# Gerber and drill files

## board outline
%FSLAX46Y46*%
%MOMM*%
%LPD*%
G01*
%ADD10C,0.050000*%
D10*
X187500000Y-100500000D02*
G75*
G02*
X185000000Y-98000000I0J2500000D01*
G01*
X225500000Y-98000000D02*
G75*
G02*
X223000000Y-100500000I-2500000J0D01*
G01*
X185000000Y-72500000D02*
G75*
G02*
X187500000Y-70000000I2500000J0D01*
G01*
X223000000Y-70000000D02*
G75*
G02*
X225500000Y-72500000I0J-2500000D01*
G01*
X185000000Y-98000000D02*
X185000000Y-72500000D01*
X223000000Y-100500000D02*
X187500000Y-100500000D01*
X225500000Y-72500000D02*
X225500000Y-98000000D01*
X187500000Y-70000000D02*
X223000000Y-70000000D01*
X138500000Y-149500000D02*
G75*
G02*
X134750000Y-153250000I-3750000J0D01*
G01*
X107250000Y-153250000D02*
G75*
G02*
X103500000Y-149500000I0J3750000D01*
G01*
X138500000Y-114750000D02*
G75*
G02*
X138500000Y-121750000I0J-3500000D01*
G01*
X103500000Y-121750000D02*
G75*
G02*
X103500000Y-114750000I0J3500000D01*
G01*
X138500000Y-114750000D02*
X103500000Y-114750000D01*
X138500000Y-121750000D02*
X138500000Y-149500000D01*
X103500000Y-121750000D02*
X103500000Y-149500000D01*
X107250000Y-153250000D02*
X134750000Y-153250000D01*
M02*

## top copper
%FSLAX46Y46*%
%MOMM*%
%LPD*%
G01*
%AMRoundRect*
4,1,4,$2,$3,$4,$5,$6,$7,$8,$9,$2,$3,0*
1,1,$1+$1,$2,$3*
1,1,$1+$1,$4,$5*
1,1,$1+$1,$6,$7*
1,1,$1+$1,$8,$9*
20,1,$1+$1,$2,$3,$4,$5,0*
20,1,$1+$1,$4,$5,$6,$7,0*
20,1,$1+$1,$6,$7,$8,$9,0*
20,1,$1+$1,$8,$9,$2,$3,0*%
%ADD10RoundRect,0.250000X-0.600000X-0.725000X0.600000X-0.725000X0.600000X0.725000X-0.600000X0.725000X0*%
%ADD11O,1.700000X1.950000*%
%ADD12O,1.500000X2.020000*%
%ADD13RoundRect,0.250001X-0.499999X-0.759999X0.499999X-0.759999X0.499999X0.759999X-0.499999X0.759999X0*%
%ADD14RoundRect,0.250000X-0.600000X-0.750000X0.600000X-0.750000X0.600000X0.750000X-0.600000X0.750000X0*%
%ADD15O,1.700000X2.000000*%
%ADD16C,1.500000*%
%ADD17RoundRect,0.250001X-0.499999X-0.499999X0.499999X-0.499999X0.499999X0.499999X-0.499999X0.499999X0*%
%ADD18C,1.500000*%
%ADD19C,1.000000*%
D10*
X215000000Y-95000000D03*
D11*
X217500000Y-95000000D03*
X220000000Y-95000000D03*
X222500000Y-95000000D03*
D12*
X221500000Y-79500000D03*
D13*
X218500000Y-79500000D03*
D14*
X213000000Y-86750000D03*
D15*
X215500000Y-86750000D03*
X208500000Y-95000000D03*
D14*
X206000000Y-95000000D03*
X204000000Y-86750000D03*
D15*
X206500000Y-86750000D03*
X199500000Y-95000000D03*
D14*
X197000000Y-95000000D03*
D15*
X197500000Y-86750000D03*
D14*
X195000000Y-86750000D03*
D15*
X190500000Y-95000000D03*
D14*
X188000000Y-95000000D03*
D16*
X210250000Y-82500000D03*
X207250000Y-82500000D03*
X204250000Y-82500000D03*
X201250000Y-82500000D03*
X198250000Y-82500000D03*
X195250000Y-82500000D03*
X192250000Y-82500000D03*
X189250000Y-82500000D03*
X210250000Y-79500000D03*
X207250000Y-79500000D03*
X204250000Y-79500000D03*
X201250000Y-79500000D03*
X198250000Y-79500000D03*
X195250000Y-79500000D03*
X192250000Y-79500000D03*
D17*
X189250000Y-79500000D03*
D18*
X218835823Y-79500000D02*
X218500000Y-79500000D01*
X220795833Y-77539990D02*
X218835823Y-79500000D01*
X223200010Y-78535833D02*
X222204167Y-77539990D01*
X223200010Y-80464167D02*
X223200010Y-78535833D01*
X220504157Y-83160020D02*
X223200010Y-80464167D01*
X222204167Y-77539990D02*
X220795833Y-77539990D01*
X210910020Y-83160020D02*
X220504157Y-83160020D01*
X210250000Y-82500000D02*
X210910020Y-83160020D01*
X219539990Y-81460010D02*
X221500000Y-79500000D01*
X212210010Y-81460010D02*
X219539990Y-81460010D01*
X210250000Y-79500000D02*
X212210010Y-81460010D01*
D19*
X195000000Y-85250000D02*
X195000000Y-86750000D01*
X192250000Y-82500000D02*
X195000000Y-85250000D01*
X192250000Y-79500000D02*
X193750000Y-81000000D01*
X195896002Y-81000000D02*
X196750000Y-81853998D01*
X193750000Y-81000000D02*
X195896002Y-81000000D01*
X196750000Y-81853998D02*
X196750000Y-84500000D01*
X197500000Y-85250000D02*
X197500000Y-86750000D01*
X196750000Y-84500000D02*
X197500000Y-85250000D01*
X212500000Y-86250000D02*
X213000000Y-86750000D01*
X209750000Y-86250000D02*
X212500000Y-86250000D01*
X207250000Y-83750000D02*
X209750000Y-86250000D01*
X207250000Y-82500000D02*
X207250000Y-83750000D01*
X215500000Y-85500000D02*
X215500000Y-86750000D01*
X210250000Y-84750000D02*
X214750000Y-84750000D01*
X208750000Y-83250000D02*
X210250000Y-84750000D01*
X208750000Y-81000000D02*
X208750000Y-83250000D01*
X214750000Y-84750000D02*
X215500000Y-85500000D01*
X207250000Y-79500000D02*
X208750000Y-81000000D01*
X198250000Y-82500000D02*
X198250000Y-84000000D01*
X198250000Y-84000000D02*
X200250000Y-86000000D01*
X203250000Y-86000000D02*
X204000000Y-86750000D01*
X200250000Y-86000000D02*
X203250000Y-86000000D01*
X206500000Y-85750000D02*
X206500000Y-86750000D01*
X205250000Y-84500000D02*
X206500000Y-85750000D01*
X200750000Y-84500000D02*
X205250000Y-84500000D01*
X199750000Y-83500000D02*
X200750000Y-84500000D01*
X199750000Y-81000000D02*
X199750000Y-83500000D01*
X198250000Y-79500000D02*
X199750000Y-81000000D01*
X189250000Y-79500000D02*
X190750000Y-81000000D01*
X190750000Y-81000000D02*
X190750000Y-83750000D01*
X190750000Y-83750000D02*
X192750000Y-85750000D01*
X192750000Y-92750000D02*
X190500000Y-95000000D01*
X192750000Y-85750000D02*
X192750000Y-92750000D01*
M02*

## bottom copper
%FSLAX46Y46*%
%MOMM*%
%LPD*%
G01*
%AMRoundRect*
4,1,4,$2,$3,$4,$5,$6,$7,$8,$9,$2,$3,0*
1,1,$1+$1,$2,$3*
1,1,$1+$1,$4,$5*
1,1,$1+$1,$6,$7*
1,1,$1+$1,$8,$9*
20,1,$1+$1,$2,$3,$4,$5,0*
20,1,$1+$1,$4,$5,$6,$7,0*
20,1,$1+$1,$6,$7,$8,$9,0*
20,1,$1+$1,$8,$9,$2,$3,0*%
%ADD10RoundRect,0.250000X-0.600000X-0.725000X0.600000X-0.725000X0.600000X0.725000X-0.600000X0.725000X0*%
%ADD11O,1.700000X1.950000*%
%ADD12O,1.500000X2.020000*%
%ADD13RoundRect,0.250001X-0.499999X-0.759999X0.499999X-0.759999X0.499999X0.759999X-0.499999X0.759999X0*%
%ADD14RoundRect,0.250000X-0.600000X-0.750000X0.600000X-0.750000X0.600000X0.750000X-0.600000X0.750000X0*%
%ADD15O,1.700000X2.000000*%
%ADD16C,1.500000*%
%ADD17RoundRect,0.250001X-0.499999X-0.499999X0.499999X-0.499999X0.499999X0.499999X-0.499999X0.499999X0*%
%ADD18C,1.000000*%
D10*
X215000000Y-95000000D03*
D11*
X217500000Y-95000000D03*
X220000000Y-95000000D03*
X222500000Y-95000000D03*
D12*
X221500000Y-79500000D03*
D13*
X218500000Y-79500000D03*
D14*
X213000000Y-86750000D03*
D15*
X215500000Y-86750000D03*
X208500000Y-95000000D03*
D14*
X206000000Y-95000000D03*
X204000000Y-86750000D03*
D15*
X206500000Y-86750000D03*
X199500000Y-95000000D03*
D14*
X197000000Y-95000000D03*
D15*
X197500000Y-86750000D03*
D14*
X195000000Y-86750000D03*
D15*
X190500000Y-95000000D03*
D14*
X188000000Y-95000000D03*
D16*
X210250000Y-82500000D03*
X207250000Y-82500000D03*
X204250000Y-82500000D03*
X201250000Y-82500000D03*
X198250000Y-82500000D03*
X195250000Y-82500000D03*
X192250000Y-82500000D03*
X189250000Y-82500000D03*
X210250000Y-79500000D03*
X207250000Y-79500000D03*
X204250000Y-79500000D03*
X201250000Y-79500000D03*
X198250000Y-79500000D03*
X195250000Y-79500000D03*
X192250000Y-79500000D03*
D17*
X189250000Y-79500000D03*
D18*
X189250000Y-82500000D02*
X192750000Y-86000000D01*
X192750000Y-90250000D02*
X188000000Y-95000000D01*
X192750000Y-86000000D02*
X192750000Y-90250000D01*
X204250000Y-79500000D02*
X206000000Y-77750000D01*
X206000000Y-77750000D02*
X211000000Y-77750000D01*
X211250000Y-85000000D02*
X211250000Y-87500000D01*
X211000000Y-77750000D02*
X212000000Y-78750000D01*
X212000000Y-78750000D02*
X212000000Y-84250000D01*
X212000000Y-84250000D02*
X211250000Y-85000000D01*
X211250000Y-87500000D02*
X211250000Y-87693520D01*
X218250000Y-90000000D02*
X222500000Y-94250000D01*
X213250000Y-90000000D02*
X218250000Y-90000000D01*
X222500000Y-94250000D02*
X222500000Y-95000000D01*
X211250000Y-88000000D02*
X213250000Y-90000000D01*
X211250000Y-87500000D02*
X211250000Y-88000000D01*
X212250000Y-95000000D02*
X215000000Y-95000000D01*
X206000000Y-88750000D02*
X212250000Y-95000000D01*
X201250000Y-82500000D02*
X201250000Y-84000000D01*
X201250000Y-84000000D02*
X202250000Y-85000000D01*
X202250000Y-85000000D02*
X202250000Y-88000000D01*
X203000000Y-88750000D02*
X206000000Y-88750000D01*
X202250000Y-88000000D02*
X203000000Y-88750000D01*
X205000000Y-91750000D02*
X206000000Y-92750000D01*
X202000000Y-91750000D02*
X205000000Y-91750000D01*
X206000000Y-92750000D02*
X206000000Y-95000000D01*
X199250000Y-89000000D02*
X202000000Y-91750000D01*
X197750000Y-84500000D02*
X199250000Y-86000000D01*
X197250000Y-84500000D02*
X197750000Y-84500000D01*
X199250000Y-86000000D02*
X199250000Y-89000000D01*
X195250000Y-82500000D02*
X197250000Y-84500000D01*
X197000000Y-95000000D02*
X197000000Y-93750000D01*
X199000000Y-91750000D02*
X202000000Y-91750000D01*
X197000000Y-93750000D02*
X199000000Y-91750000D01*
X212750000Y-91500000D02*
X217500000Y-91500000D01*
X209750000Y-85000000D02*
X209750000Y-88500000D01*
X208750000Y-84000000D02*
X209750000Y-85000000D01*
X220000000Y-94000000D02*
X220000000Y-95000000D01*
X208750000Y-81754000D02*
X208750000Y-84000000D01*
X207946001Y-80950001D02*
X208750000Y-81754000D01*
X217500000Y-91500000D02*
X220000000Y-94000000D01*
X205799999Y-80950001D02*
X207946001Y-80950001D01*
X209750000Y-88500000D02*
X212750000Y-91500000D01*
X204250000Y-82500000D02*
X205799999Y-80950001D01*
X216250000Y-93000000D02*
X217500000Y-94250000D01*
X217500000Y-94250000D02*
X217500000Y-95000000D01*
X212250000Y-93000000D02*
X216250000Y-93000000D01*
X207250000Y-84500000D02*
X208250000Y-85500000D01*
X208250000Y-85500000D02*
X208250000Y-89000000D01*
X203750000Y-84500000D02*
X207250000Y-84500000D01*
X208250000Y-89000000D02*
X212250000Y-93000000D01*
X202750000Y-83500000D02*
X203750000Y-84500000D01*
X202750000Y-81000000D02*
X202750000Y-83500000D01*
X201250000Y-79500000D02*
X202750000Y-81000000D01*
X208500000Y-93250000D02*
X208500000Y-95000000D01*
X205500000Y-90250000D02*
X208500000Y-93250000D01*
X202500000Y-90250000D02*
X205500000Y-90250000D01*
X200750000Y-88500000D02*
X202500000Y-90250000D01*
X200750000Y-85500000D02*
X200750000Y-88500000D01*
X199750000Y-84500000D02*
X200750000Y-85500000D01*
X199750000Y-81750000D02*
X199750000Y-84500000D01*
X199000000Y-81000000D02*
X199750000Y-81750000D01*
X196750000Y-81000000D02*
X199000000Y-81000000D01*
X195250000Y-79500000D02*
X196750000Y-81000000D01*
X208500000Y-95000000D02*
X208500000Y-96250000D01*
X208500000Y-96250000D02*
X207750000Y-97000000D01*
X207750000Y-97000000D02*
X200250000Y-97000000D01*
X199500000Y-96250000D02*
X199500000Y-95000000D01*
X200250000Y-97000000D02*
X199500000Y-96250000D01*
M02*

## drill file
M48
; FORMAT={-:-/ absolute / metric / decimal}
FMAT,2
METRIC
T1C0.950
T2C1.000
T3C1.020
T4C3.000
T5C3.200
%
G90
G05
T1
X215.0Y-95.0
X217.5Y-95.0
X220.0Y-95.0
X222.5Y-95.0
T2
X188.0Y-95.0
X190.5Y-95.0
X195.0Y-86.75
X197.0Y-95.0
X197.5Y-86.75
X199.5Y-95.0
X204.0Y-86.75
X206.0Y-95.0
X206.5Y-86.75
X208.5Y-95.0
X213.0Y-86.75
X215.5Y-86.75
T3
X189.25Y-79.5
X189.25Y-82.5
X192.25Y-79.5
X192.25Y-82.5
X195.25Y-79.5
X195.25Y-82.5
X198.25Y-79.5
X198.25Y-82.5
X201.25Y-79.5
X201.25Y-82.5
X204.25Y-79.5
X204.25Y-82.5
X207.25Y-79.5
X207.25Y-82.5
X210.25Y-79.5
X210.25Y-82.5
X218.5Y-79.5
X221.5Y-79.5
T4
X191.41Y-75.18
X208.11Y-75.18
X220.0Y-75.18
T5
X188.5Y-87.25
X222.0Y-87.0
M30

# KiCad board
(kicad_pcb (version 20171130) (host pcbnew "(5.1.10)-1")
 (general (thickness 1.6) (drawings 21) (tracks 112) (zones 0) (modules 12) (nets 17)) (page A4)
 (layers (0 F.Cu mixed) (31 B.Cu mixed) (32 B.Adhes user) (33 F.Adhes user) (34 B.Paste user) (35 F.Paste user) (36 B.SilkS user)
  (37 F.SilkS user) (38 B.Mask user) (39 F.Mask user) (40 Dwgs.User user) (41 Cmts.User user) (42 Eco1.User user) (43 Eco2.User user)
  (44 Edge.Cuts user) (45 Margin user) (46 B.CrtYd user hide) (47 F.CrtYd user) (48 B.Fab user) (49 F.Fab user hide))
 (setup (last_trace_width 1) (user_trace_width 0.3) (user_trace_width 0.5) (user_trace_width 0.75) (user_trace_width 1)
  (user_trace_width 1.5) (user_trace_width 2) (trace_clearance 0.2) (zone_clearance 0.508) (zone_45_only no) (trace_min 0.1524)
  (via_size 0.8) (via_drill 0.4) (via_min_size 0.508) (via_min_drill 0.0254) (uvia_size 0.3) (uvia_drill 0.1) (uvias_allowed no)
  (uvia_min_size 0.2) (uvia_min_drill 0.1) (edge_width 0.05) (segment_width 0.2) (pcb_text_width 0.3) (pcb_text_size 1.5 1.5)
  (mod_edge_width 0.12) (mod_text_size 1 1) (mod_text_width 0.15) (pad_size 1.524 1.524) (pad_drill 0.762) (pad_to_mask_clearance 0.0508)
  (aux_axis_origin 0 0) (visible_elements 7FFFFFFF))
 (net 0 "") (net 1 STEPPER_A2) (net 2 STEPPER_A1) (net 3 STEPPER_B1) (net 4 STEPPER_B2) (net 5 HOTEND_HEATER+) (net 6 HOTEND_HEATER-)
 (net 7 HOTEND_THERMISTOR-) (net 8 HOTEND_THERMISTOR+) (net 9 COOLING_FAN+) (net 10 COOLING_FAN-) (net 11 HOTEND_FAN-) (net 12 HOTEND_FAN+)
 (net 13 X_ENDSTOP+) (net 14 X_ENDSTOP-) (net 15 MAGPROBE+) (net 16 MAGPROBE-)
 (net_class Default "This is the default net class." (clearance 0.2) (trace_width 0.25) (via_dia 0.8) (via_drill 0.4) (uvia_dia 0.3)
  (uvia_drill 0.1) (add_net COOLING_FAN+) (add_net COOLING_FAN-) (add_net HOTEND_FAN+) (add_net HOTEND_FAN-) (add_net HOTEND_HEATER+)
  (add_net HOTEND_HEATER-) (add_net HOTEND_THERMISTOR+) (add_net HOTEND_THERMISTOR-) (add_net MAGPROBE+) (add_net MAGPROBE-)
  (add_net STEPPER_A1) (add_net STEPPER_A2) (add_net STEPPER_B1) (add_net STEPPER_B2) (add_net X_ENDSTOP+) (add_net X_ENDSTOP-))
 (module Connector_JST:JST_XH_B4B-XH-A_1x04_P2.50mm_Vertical (layer F.Cu) (at 215 95)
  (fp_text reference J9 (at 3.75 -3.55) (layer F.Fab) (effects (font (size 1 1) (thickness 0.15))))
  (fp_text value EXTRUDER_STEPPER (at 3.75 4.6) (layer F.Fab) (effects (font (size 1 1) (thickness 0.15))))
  (pad 1 thru_hole roundrect (at 0 0) (size 1.7 1.95) (drill 0.95) (layers *.Cu *.Mask) (roundrect_rratio 0.147059) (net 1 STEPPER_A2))
  (pad 2 thru_hole oval (at 2.5 0) (size 1.7 1.95) (drill 0.95) (layers *.Cu *.Mask) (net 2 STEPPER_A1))
  (pad 3 thru_hole oval (at 5 0) (size 1.7 1.95) (drill 0.95) (layers *.Cu *.Mask) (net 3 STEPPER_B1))
  (pad 4 thru_hole oval (at 7.5 0) (size 1.7 1.95) (drill 0.95) (layers *.Cu *.Mask) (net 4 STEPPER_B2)))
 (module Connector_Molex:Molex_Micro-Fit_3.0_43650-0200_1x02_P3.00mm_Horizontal (layer F.Cu) (at 218.5 79.5)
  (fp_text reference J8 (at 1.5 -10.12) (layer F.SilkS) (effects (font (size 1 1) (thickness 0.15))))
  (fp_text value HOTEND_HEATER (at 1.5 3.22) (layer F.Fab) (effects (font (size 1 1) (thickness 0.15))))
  (pad 2 thru_hole oval (at 3 0) (size 1.5 2.02) (drill 1.02) (layers *.Cu *.Mask) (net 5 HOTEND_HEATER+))
  (pad 1 thru_hole roundrect (at 0 0) (size 1.5 2.02) (drill 1.02) (layers *.Cu *.Mask) (roundrect_rratio 0.166667) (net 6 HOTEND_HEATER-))
  (pad "" np_thru_hole circle (at 1.5 -4.32) (size 3 3) (drill 3) (layers *.Cu *.Mask)))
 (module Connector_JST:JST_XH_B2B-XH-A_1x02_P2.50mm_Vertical (layer F.Cu) (at 213 86.75)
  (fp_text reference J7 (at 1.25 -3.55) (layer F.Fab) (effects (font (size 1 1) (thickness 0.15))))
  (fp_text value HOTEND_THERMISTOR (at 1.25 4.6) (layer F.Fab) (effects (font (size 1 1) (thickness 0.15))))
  (pad 1 thru_hole roundrect (at 0 0) (size 1.7 2) (drill 1) (layers *.Cu *.Mask) (roundrect_rratio 0.147059) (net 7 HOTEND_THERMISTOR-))
  (pad 2 thru_hole oval (at 2.5 0) (size 1.7 2) (drill 1) (layers *.Cu *.Mask) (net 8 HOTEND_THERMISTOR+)))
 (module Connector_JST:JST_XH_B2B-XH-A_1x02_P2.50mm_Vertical (layer F.Cu) (at 206 95)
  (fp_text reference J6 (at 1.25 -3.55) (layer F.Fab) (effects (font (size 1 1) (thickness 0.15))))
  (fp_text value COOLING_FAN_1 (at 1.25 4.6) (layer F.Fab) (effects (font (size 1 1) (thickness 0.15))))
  (pad 2 thru_hole oval (at 2.5 0) (size 1.7 2) (drill 1) (layers *.Cu *.Mask) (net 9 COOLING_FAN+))
  (pad 1 thru_hole roundrect (at 0 0) (size 1.7 2) (drill 1) (layers *.Cu *.Mask) (roundrect_rratio 0.147059) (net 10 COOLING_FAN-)))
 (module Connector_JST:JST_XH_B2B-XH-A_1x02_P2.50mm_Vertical (layer F.Cu) (at 204 86.75)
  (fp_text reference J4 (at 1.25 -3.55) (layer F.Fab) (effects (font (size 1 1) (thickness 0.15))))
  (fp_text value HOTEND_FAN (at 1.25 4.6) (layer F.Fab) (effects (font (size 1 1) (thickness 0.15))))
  (pad 1 thru_hole roundrect (at 0 0) (size 1.7 2) (drill 1) (layers *.Cu *.Mask) (roundrect_rratio 0.147059) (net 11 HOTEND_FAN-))
  (pad 2 thru_hole oval (at 2.5 0) (size 1.7 2) (drill 1) (layers *.Cu *.Mask) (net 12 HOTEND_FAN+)))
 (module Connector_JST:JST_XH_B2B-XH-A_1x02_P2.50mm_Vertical (layer F.Cu) (at 197 95)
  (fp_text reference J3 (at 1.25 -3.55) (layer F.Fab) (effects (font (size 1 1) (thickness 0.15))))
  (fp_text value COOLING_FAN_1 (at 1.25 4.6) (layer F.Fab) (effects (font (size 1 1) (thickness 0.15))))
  (pad 2 thru_hole oval (at 2.5 0) (size 1.7 2) (drill 1) (layers *.Cu *.Mask) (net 9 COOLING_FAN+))
  (pad 1 thru_hole roundrect (at 0 0) (size 1.7 2) (drill 1) (layers *.Cu *.Mask) (roundrect_rratio 0.147059) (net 10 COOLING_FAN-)))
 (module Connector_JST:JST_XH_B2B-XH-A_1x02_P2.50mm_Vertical (layer F.Cu) (at 195 86.75)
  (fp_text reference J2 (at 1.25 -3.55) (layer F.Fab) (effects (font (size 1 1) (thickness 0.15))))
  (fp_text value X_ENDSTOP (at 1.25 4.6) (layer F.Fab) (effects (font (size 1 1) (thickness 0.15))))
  (pad 2 thru_hole oval (at 2.5 0) (size 1.7 2) (drill 1) (layers *.Cu *.Mask) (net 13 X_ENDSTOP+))
  (pad 1 thru_hole roundrect (at 0 0) (size 1.7 2) (drill 1) (layers *.Cu *.Mask) (roundrect_rratio 0.147059) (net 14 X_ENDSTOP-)))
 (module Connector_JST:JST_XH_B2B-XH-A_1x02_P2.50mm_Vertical (layer F.Cu) (at 188 95)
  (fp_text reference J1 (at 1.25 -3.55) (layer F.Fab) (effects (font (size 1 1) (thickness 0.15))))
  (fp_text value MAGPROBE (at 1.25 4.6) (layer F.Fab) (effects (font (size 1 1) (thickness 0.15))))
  (pad 2 thru_hole oval (at 2.5 0) (size 1.7 2) (drill 1) (layers *.Cu *.Mask) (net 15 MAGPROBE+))
  (pad 1 thru_hole roundrect (at 0 0) (size 1.7 2) (drill 1) (layers *.Cu *.Mask) (roundrect_rratio 0.147059) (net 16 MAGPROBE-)))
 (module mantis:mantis (layer F.Cu) (at 94.25 131.5)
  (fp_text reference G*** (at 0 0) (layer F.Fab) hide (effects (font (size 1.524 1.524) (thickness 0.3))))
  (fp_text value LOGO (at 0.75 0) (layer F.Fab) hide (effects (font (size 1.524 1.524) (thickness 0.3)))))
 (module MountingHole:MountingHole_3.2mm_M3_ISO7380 (layer F.Cu) (at 188.5 87.25)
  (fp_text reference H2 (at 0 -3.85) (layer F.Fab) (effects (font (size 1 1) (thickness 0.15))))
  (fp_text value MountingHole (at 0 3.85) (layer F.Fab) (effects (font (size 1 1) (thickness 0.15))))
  (pad 1 np_thru_hole circle (at 0 0) (size 3.2 3.2) (drill 3.2) (layers *.Cu *.Mask)))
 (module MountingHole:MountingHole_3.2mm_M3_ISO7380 (layer F.Cu) (at 222 87)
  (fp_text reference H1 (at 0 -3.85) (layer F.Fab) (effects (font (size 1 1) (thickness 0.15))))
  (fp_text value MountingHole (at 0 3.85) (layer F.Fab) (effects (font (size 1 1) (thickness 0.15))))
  (pad 1 np_thru_hole circle (at 0 0) (size 3.2 3.2) (drill 3.2) (layers *.Cu *.Mask)))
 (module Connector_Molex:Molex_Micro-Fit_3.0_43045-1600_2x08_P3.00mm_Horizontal (layer F.Cu) (at 189.25 79.5)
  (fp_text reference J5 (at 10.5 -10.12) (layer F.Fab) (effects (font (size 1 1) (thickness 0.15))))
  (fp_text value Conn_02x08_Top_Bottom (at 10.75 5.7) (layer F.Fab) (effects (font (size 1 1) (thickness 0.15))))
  (pad 16 thru_hole circle (at 21 3) (size 1.5 1.5) (drill 1.02) (layers *.Cu *.Mask) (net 6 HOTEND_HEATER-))
  (pad 15 thru_hole circle (at 18 3) (size 1.5 1.5) (drill 1.02) (layers *.Cu *.Mask) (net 7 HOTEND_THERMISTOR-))
  (pad 14 thru_hole circle (at 15 3) (size 1.5 1.5) (drill 1.02) (layers *.Cu *.Mask) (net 3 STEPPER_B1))
  (pad 13 thru_hole circle (at 12 3) (size 1.5 1.5) (drill 1.02) (layers *.Cu *.Mask) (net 1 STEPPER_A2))
  (pad 12 thru_hole circle (at 9 3) (size 1.5 1.5) (drill 1.02) (layers *.Cu *.Mask) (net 11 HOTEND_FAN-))
  (pad 11 thru_hole circle (at 6 3) (size 1.5 1.5) (drill 1.02) (layers *.Cu *.Mask) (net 10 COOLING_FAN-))
  (pad 10 thru_hole circle (at 3 3) (size 1.5 1.5) (drill 1.02) (layers *.Cu *.Mask) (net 14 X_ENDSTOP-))
  (pad 9 thru_hole circle (at 0 3) (size 1.5 1.5) (drill 1.02) (layers *.Cu *.Mask) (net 16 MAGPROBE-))
  (pad 8 thru_hole circle (at 21 0) (size 1.5 1.5) (drill 1.02) (layers *.Cu *.Mask) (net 5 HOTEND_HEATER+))
  (pad 7 thru_hole circle (at 18 0) (size 1.5 1.5) (drill 1.02) (layers *.Cu *.Mask) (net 8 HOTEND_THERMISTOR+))
  (pad 6 thru_hole circle (at 15 0) (size 1.5 1.5) (drill 1.02) (layers *.Cu *.Mask) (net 4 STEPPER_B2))
  (pad 5 thru_hole circle (at 12 0) (size 1.5 1.5) (drill 1.02) (layers *.Cu *.Mask) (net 2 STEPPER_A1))
  (pad 4 thru_hole circle (at 9 0) (size 1.5 1.5) (drill 1.02) (layers *.Cu *.Mask) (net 12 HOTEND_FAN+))
  (pad 3 thru_hole circle (at 6 0) (size 1.5 1.5) (drill 1.02) (layers *.Cu *.Mask) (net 9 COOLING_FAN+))
  (pad 2 thru_hole circle (at 3 0) (size 1.5 1.5) (drill 1.02) (layers *.Cu *.Mask) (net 13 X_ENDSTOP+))
  (pad 1 thru_hole roundrect (at 0 0) (size 1.5 1.5) (drill 1.02) (layers *.Cu *.Mask) (roundrect_rratio 0.166667) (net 15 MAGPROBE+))
  (pad "" np_thru_hole circle (at 18.86 -4.32) (size 3 3) (drill 3) (layers *.Cu *.Mask))
  (pad "" np_thru_hole circle (at 2.16 -4.32) (size 3 3) (drill 3) (layers *.Cu *.Mask)))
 (gr_arc (start 187.5 98) (end 185 98) (angle -90) (layer Edge.Cuts) (width 0.05))
 (gr_arc (start 223 98) (end 223 100.5) (angle -90) (layer Edge.Cuts) (width 0.05))
 (gr_arc (start 187.5 72.5) (end 187.5 70) (angle -90) (layer Edge.Cuts) (width 0.05))
 (gr_arc (start 223 72.5) (end 225.5 72.5) (angle -90) (layer Edge.Cuts) (width 0.05))
 (gr_line (start 185 98) (end 185 72.5) (layer Edge.Cuts) (width 0.05))
 (gr_line (start 223 100.5) (end 187.5 100.5) (layer Edge.Cuts) (width 0.05))
 (gr_line (start 225.5 72.5) (end 225.5 98) (layer Edge.Cuts) (width 0.05))
 (gr_line (start 187.5 70) (end 223 70) (layer Edge.Cuts) (width 0.05))
 (gr_arc (start 134.75 149.5) (end 134.75 153.25) (angle -90) (layer Edge.Cuts) (width 0.05))
 (gr_arc (start 107.25 149.5) (end 103.5 149.5) (angle -90) (layer Edge.Cuts) (width 0.05))
 (gr_arc (start 138.5 118.25) (end 138.5 121.75) (angle -180) (layer Edge.Cuts) (width 0.05))
 (gr_arc (start 103.5 118.25) (end 103.5 114.75) (angle -180) (layer Edge.Cuts) (width 0.05))
 (gr_line (start 138.5 114.75) (end 103.5 114.75) (layer Edge.Cuts) (width 0.05))
 (gr_line (start 138.5 121.75) (end 138.5 149.5) (layer Edge.Cuts) (width 0.05))
 (gr_line (start 103.5 121.75) (end 103.5 149.5) (layer Edge.Cuts) (width 0.05))
 (gr_line (start 107.25 153.25) (end 134.75 153.25) (layer Edge.Cuts) (width 0.05))
 (segment (start 218.835823 79.5) (end 218.5 79.5) (width 1.5) (layer F.Cu) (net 6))
 (segment (start 220.795833 77.53999) (end 218.835823 79.5) (width 1.5) (layer F.Cu) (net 6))
 (segment (start 223.20001 78.535833) (end 222.204167 77.53999) (width 1.5) (layer F.Cu) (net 6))
 (segment (start 223.20001 80.464167) (end 223.20001 78.535833) (width 1.5) (layer F.Cu) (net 6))
 (segment (start 220.504157 83.16002) (end 223.20001 80.464167) (width 1.5) (layer F.Cu) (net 6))
 (segment (start 222.204167 77.53999) (end 220.795833 77.53999) (width 1.5) (layer F.Cu) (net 6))
 (segment (start 210.91002 83.16002) (end 220.504157 83.16002) (width 1.5) (layer F.Cu) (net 6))
 (segment (start 210.25 82.5) (end 210.91002 83.16002) (width 1.5) (layer F.Cu) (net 6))
 (segment (start 219.53999 81.46001) (end 221.5 79.5) (width 1.5) (layer F.Cu) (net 5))
 (segment (start 212.21001 81.46001) (end 219.53999 81.46001) (width 1.5) (layer F.Cu) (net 5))
 (segment (start 210.25 79.5) (end 212.21001 81.46001) (width 1.5) (layer F.Cu) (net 5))
 (segment (start 195 85.25) (end 195 86.75) (width 1) (layer F.Cu) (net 14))
 (segment (start 192.25 82.5) (end 195 85.25) (width 1) (layer F.Cu) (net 14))
 (segment (start 192.25 79.5) (end 193.75 81) (width 1) (layer F.Cu) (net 13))
 (segment (start 195.896002 81) (end 196.75 81.853998) (width 1) (layer F.Cu) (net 13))
 (segment (start 193.75 81) (end 195.896002 81) (width 1) (layer F.Cu) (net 13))
 (segment (start 196.75 81.853998) (end 196.75 84.5) (width 1) (layer F.Cu) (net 13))
 (segment (start 197.5 85.25) (end 197.5 86.75) (width 1) (layer F.Cu) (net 13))
 (segment (start 196.75 84.5) (end 197.5 85.25) (width 1) (layer F.Cu) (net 13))
 (segment (start 212.5 86.25) (end 213 86.75) (width 1) (layer F.Cu) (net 7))
 (segment (start 209.75 86.25) (end 212.5 86.25) (width 1) (layer F.Cu) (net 7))
 (segment (start 207.25 83.75) (end 209.75 86.25) (width 1) (layer F.Cu) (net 7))
 (segment (start 207.25 82.5) (end 207.25 83.75) (width 1) (layer F.Cu) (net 7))
 (segment (start 215.5 85.5) (end 215.5 86.75) (width 1) (layer F.Cu) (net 8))
 (segment (start 210.25 84.75) (end 214.75 84.75) (width 1) (layer F.Cu) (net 8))
 (segment (start 208.75 83.25) (end 210.25 84.75) (width 1) (layer F.Cu) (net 8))
 (segment (start 208.75 81) (end 208.75 83.25) (width 1) (layer F.Cu) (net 8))
 (segment (start 214.75 84.75) (end 215.5 85.5) (width 1) (layer F.Cu) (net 8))
 (segment (start 207.25 79.5) (end 208.75 81) (width 1) (layer F.Cu) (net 8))
 (segment (start 198.25 82.5) (end 198.25 84) (width 1) (layer F.Cu) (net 11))
 (segment (start 198.25 84) (end 200.25 86) (width 1) (layer F.Cu) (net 11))
 (segment (start 203.25 86) (end 204 86.75) (width 1) (layer F.Cu) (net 11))
 (segment (start 200.25 86) (end 203.25 86) (width 1) (layer F.Cu) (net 11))
 (segment (start 206.5 85.75) (end 206.5 86.75) (width 1) (layer F.Cu) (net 12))
 (segment (start 205.25 84.5) (end 206.5 85.75) (width 1) (layer F.Cu) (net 12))
 (segment (start 200.75 84.5) (end 205.25 84.5) (width 1) (layer F.Cu) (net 12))
 (segment (start 199.75 83.5) (end 200.75 84.5) (width 1) (layer F.Cu) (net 12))
 (segment (start 199.75 81) (end 199.75 83.5) (width 1) (layer F.Cu) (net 12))
 (segment (start 198.25 79.5) (end 199.75 81) (width 1) (layer F.Cu) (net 12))
 (segment (start 189.25 82.5) (end 192.75 86) (width 1) (layer B.Cu) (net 16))
 (segment (start 192.75 90.25) (end 188 95) (width 1) (layer B.Cu) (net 16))
 (segment (start 192.75 86) (end 192.75 90.25) (width 1) (layer B.Cu) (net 16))
 (segment (start 204.25 79.5) (end 206 77.75) (width 1) (layer B.Cu) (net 4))
 (segment (start 206 77.75) (end 211 77.75) (width 1) (layer B.Cu) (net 4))
 (segment (start 211.25 85) (end 211.25 87.5) (width 1) (layer B.Cu) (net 4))
 (segment (start 211 77.75) (end 212 78.75) (width 1) (layer B.Cu) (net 4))
 (segment (start 212 78.75) (end 212 84.25) (width 1) (layer B.Cu) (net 4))
 (segment (start 212 84.25) (end 211.25 85) (width 1) (layer B.Cu) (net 4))
 (segment (start 211.25 87.5) (end 211.25 87.69352) (width 1) (layer B.Cu) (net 4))
 (segment (start 218.25 90) (end 222.5 94.25) (width 1) (layer B.Cu) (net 4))
 (segment (start 213.25 90) (end 218.25 90) (width 1) (layer B.Cu) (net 4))
 (segment (start 222.5 94.25) (end 222.5 95) (width 1) (layer B.Cu) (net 4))
 (segment (start 211.25 88) (end 213.25 90) (width 1) (layer B.Cu) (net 4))
 (segment (start 211.25 87.5) (end 211.25 88) (width 1) (layer B.Cu) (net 4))
 (segment (start 212.25 95) (end 215 95) (width 1) (layer B.Cu) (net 1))
 (segment (start 206 88.75) (end 212.25 95) (width 1) (layer B.Cu) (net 1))
 (segment (start 201.25 82.5) (end 201.25 84) (width 1) (layer B.Cu) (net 1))
 (segment (start 201.25 84) (end 202.25 85) (width 1) (layer B.Cu) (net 1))
 (segment (start 202.25 85) (end 202.25 88) (width 1) (layer B.Cu) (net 1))
 (segment (start 203 88.75) (end 206 88.75) (width 1) (layer B.Cu) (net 1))
 (segment (start 202.25 88) (end 203 88.75) (width 1) (layer B.Cu) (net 1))
 (segment (start 205 91.75) (end 206 92.75) (width 1) (layer B.Cu) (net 10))
 (segment (start 202 91.75) (end 205 91.75) (width 1) (layer B.Cu) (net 10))
 (segment (start 206 92.75) (end 206 95) (width 1) (layer B.Cu) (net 10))
 (segment (start 199.25 89) (end 202 91.75) (width 1) (layer B.Cu) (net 10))
 (segment (start 197.75 84.5) (end 199.25 86) (width 1) (layer B.Cu) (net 10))
 (segment (start 197.25 84.5) (end 197.75 84.5) (width 1) (layer B.Cu) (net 10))
 (segment (start 199.25 86) (end 199.25 89) (width 1) (layer B.Cu) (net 10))
 (segment (start 195.25 82.5) (end 197.25 84.5) (width 1) (layer B.Cu) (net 10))
 (segment (start 197 95) (end 197 93.75) (width 1) (layer B.Cu) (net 10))
 (segment (start 199 91.75) (end 202 91.75) (width 1) (layer B.Cu) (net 10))
 (segment (start 197 93.75) (end 199 91.75) (width 1) (layer B.Cu) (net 10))
 (segment (start 189.25 79.5) (end 190.75 81) (width 1) (layer F.Cu) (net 15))
 (segment (start 190.75 81) (end 190.75 83.75) (width 1) (layer F.Cu) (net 15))
 (segment (start 190.75 83.75) (end 192.75 85.75) (width 1) (layer F.Cu) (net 15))
 (segment (start 192.75 92.75) (end 190.5 95) (width 1) (layer F.Cu) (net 15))
 (segment (start 192.75 85.75) (end 192.75 92.75) (width 1) (layer F.Cu) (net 15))
 (segment (start 212.75 91.5) (end 217.5 91.5) (width 1) (layer B.Cu) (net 3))
 (segment (start 209.75 85) (end 209.75 88.5) (width 1) (layer B.Cu) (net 3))
 (segment (start 208.75 84) (end 209.75 85) (width 1) (layer B.Cu) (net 3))
 (segment (start 220 94) (end 220 95) (width 1) (layer B.Cu) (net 3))
 (segment (start 208.75 81.754) (end 208.75 84) (width 1) (layer B.Cu) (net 3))
 (segment (start 207.946001 80.950001) (end 208.75 81.754) (width 1) (layer B.Cu) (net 3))
 (segment (start 217.5 91.5) (end 220 94) (width 1) (layer B.Cu) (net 3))
 (segment (start 205.799999 80.950001) (end 207.946001 80.950001) (width 1) (layer B.Cu) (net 3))
 (segment (start 209.75 88.5) (end 212.75 91.5) (width 1) (layer B.Cu) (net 3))
 (segment (start 204.25 82.5) (end 205.799999 80.950001) (width 1) (layer B.Cu) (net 3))
 (segment (start 216.25 93) (end 217.5 94.25) (width 1) (layer B.Cu) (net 2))
 (segment (start 217.5 94.25) (end 217.5 95) (width 1) (layer B.Cu) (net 2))
 (segment (start 212.25 93) (end 216.25 93) (width 1) (layer B.Cu) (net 2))
 (segment (start 207.25 84.5) (end 208.25 85.5) (width 1) (layer B.Cu) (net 2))
 (segment (start 208.25 85.5) (end 208.25 89) (width 1) (layer B.Cu) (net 2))
 (segment (start 203.75 84.5) (end 207.25 84.5) (width 1) (layer B.Cu) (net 2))
 (segment (start 208.25 89) (end 212.25 93) (width 1) (layer B.Cu) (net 2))
 (segment (start 202.75 83.5) (end 203.75 84.5) (width 1) (layer B.Cu) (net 2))
 (segment (start 202.75 81) (end 202.75 83.5) (width 1) (layer B.Cu) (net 2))
 (segment (start 201.25 79.5) (end 202.75 81) (width 1) (layer B.Cu) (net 2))
 (segment (start 208.5 93.25) (end 208.5 95) (width 1) (layer B.Cu) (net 9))
 (segment (start 205.5 90.25) (end 208.5 93.25) (width 1) (layer B.Cu) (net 9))
 (segment (start 202.5 90.25) (end 205.5 90.25) (width 1) (layer B.Cu) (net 9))
 (segment (start 200.75 88.5) (end 202.5 90.25) (width 1) (layer B.Cu) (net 9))
 (segment (start 200.75 85.5) (end 200.75 88.5) (width 1) (layer B.Cu) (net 9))
 (segment (start 199.75 84.5) (end 200.75 85.5) (width 1) (layer B.Cu) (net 9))
 (segment (start 199.75 81.75) (end 199.75 84.5) (width 1) (layer B.Cu) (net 9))
 (segment (start 199 81) (end 199.75 81.75) (width 1) (layer B.Cu) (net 9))
 (segment (start 196.75 81) (end 199 81) (width 1) (layer B.Cu) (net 9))
 (segment (start 195.25 79.5) (end 196.75 81) (width 1) (layer B.Cu) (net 9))
 (segment (start 208.5 95) (end 208.5 96.25) (width 1) (layer B.Cu) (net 9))
 (segment (start 208.5 96.25) (end 207.75 97) (width 1) (layer B.Cu) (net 9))
 (segment (start 207.75 97) (end 200.25 97) (width 1) (layer B.Cu) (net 9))
 (segment (start 199.5 96.25) (end 199.5 95) (width 1) (layer B.Cu) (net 9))
 (segment (start 200.25 97) (end 199.5 96.25) (width 1) (layer B.Cu) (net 9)))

